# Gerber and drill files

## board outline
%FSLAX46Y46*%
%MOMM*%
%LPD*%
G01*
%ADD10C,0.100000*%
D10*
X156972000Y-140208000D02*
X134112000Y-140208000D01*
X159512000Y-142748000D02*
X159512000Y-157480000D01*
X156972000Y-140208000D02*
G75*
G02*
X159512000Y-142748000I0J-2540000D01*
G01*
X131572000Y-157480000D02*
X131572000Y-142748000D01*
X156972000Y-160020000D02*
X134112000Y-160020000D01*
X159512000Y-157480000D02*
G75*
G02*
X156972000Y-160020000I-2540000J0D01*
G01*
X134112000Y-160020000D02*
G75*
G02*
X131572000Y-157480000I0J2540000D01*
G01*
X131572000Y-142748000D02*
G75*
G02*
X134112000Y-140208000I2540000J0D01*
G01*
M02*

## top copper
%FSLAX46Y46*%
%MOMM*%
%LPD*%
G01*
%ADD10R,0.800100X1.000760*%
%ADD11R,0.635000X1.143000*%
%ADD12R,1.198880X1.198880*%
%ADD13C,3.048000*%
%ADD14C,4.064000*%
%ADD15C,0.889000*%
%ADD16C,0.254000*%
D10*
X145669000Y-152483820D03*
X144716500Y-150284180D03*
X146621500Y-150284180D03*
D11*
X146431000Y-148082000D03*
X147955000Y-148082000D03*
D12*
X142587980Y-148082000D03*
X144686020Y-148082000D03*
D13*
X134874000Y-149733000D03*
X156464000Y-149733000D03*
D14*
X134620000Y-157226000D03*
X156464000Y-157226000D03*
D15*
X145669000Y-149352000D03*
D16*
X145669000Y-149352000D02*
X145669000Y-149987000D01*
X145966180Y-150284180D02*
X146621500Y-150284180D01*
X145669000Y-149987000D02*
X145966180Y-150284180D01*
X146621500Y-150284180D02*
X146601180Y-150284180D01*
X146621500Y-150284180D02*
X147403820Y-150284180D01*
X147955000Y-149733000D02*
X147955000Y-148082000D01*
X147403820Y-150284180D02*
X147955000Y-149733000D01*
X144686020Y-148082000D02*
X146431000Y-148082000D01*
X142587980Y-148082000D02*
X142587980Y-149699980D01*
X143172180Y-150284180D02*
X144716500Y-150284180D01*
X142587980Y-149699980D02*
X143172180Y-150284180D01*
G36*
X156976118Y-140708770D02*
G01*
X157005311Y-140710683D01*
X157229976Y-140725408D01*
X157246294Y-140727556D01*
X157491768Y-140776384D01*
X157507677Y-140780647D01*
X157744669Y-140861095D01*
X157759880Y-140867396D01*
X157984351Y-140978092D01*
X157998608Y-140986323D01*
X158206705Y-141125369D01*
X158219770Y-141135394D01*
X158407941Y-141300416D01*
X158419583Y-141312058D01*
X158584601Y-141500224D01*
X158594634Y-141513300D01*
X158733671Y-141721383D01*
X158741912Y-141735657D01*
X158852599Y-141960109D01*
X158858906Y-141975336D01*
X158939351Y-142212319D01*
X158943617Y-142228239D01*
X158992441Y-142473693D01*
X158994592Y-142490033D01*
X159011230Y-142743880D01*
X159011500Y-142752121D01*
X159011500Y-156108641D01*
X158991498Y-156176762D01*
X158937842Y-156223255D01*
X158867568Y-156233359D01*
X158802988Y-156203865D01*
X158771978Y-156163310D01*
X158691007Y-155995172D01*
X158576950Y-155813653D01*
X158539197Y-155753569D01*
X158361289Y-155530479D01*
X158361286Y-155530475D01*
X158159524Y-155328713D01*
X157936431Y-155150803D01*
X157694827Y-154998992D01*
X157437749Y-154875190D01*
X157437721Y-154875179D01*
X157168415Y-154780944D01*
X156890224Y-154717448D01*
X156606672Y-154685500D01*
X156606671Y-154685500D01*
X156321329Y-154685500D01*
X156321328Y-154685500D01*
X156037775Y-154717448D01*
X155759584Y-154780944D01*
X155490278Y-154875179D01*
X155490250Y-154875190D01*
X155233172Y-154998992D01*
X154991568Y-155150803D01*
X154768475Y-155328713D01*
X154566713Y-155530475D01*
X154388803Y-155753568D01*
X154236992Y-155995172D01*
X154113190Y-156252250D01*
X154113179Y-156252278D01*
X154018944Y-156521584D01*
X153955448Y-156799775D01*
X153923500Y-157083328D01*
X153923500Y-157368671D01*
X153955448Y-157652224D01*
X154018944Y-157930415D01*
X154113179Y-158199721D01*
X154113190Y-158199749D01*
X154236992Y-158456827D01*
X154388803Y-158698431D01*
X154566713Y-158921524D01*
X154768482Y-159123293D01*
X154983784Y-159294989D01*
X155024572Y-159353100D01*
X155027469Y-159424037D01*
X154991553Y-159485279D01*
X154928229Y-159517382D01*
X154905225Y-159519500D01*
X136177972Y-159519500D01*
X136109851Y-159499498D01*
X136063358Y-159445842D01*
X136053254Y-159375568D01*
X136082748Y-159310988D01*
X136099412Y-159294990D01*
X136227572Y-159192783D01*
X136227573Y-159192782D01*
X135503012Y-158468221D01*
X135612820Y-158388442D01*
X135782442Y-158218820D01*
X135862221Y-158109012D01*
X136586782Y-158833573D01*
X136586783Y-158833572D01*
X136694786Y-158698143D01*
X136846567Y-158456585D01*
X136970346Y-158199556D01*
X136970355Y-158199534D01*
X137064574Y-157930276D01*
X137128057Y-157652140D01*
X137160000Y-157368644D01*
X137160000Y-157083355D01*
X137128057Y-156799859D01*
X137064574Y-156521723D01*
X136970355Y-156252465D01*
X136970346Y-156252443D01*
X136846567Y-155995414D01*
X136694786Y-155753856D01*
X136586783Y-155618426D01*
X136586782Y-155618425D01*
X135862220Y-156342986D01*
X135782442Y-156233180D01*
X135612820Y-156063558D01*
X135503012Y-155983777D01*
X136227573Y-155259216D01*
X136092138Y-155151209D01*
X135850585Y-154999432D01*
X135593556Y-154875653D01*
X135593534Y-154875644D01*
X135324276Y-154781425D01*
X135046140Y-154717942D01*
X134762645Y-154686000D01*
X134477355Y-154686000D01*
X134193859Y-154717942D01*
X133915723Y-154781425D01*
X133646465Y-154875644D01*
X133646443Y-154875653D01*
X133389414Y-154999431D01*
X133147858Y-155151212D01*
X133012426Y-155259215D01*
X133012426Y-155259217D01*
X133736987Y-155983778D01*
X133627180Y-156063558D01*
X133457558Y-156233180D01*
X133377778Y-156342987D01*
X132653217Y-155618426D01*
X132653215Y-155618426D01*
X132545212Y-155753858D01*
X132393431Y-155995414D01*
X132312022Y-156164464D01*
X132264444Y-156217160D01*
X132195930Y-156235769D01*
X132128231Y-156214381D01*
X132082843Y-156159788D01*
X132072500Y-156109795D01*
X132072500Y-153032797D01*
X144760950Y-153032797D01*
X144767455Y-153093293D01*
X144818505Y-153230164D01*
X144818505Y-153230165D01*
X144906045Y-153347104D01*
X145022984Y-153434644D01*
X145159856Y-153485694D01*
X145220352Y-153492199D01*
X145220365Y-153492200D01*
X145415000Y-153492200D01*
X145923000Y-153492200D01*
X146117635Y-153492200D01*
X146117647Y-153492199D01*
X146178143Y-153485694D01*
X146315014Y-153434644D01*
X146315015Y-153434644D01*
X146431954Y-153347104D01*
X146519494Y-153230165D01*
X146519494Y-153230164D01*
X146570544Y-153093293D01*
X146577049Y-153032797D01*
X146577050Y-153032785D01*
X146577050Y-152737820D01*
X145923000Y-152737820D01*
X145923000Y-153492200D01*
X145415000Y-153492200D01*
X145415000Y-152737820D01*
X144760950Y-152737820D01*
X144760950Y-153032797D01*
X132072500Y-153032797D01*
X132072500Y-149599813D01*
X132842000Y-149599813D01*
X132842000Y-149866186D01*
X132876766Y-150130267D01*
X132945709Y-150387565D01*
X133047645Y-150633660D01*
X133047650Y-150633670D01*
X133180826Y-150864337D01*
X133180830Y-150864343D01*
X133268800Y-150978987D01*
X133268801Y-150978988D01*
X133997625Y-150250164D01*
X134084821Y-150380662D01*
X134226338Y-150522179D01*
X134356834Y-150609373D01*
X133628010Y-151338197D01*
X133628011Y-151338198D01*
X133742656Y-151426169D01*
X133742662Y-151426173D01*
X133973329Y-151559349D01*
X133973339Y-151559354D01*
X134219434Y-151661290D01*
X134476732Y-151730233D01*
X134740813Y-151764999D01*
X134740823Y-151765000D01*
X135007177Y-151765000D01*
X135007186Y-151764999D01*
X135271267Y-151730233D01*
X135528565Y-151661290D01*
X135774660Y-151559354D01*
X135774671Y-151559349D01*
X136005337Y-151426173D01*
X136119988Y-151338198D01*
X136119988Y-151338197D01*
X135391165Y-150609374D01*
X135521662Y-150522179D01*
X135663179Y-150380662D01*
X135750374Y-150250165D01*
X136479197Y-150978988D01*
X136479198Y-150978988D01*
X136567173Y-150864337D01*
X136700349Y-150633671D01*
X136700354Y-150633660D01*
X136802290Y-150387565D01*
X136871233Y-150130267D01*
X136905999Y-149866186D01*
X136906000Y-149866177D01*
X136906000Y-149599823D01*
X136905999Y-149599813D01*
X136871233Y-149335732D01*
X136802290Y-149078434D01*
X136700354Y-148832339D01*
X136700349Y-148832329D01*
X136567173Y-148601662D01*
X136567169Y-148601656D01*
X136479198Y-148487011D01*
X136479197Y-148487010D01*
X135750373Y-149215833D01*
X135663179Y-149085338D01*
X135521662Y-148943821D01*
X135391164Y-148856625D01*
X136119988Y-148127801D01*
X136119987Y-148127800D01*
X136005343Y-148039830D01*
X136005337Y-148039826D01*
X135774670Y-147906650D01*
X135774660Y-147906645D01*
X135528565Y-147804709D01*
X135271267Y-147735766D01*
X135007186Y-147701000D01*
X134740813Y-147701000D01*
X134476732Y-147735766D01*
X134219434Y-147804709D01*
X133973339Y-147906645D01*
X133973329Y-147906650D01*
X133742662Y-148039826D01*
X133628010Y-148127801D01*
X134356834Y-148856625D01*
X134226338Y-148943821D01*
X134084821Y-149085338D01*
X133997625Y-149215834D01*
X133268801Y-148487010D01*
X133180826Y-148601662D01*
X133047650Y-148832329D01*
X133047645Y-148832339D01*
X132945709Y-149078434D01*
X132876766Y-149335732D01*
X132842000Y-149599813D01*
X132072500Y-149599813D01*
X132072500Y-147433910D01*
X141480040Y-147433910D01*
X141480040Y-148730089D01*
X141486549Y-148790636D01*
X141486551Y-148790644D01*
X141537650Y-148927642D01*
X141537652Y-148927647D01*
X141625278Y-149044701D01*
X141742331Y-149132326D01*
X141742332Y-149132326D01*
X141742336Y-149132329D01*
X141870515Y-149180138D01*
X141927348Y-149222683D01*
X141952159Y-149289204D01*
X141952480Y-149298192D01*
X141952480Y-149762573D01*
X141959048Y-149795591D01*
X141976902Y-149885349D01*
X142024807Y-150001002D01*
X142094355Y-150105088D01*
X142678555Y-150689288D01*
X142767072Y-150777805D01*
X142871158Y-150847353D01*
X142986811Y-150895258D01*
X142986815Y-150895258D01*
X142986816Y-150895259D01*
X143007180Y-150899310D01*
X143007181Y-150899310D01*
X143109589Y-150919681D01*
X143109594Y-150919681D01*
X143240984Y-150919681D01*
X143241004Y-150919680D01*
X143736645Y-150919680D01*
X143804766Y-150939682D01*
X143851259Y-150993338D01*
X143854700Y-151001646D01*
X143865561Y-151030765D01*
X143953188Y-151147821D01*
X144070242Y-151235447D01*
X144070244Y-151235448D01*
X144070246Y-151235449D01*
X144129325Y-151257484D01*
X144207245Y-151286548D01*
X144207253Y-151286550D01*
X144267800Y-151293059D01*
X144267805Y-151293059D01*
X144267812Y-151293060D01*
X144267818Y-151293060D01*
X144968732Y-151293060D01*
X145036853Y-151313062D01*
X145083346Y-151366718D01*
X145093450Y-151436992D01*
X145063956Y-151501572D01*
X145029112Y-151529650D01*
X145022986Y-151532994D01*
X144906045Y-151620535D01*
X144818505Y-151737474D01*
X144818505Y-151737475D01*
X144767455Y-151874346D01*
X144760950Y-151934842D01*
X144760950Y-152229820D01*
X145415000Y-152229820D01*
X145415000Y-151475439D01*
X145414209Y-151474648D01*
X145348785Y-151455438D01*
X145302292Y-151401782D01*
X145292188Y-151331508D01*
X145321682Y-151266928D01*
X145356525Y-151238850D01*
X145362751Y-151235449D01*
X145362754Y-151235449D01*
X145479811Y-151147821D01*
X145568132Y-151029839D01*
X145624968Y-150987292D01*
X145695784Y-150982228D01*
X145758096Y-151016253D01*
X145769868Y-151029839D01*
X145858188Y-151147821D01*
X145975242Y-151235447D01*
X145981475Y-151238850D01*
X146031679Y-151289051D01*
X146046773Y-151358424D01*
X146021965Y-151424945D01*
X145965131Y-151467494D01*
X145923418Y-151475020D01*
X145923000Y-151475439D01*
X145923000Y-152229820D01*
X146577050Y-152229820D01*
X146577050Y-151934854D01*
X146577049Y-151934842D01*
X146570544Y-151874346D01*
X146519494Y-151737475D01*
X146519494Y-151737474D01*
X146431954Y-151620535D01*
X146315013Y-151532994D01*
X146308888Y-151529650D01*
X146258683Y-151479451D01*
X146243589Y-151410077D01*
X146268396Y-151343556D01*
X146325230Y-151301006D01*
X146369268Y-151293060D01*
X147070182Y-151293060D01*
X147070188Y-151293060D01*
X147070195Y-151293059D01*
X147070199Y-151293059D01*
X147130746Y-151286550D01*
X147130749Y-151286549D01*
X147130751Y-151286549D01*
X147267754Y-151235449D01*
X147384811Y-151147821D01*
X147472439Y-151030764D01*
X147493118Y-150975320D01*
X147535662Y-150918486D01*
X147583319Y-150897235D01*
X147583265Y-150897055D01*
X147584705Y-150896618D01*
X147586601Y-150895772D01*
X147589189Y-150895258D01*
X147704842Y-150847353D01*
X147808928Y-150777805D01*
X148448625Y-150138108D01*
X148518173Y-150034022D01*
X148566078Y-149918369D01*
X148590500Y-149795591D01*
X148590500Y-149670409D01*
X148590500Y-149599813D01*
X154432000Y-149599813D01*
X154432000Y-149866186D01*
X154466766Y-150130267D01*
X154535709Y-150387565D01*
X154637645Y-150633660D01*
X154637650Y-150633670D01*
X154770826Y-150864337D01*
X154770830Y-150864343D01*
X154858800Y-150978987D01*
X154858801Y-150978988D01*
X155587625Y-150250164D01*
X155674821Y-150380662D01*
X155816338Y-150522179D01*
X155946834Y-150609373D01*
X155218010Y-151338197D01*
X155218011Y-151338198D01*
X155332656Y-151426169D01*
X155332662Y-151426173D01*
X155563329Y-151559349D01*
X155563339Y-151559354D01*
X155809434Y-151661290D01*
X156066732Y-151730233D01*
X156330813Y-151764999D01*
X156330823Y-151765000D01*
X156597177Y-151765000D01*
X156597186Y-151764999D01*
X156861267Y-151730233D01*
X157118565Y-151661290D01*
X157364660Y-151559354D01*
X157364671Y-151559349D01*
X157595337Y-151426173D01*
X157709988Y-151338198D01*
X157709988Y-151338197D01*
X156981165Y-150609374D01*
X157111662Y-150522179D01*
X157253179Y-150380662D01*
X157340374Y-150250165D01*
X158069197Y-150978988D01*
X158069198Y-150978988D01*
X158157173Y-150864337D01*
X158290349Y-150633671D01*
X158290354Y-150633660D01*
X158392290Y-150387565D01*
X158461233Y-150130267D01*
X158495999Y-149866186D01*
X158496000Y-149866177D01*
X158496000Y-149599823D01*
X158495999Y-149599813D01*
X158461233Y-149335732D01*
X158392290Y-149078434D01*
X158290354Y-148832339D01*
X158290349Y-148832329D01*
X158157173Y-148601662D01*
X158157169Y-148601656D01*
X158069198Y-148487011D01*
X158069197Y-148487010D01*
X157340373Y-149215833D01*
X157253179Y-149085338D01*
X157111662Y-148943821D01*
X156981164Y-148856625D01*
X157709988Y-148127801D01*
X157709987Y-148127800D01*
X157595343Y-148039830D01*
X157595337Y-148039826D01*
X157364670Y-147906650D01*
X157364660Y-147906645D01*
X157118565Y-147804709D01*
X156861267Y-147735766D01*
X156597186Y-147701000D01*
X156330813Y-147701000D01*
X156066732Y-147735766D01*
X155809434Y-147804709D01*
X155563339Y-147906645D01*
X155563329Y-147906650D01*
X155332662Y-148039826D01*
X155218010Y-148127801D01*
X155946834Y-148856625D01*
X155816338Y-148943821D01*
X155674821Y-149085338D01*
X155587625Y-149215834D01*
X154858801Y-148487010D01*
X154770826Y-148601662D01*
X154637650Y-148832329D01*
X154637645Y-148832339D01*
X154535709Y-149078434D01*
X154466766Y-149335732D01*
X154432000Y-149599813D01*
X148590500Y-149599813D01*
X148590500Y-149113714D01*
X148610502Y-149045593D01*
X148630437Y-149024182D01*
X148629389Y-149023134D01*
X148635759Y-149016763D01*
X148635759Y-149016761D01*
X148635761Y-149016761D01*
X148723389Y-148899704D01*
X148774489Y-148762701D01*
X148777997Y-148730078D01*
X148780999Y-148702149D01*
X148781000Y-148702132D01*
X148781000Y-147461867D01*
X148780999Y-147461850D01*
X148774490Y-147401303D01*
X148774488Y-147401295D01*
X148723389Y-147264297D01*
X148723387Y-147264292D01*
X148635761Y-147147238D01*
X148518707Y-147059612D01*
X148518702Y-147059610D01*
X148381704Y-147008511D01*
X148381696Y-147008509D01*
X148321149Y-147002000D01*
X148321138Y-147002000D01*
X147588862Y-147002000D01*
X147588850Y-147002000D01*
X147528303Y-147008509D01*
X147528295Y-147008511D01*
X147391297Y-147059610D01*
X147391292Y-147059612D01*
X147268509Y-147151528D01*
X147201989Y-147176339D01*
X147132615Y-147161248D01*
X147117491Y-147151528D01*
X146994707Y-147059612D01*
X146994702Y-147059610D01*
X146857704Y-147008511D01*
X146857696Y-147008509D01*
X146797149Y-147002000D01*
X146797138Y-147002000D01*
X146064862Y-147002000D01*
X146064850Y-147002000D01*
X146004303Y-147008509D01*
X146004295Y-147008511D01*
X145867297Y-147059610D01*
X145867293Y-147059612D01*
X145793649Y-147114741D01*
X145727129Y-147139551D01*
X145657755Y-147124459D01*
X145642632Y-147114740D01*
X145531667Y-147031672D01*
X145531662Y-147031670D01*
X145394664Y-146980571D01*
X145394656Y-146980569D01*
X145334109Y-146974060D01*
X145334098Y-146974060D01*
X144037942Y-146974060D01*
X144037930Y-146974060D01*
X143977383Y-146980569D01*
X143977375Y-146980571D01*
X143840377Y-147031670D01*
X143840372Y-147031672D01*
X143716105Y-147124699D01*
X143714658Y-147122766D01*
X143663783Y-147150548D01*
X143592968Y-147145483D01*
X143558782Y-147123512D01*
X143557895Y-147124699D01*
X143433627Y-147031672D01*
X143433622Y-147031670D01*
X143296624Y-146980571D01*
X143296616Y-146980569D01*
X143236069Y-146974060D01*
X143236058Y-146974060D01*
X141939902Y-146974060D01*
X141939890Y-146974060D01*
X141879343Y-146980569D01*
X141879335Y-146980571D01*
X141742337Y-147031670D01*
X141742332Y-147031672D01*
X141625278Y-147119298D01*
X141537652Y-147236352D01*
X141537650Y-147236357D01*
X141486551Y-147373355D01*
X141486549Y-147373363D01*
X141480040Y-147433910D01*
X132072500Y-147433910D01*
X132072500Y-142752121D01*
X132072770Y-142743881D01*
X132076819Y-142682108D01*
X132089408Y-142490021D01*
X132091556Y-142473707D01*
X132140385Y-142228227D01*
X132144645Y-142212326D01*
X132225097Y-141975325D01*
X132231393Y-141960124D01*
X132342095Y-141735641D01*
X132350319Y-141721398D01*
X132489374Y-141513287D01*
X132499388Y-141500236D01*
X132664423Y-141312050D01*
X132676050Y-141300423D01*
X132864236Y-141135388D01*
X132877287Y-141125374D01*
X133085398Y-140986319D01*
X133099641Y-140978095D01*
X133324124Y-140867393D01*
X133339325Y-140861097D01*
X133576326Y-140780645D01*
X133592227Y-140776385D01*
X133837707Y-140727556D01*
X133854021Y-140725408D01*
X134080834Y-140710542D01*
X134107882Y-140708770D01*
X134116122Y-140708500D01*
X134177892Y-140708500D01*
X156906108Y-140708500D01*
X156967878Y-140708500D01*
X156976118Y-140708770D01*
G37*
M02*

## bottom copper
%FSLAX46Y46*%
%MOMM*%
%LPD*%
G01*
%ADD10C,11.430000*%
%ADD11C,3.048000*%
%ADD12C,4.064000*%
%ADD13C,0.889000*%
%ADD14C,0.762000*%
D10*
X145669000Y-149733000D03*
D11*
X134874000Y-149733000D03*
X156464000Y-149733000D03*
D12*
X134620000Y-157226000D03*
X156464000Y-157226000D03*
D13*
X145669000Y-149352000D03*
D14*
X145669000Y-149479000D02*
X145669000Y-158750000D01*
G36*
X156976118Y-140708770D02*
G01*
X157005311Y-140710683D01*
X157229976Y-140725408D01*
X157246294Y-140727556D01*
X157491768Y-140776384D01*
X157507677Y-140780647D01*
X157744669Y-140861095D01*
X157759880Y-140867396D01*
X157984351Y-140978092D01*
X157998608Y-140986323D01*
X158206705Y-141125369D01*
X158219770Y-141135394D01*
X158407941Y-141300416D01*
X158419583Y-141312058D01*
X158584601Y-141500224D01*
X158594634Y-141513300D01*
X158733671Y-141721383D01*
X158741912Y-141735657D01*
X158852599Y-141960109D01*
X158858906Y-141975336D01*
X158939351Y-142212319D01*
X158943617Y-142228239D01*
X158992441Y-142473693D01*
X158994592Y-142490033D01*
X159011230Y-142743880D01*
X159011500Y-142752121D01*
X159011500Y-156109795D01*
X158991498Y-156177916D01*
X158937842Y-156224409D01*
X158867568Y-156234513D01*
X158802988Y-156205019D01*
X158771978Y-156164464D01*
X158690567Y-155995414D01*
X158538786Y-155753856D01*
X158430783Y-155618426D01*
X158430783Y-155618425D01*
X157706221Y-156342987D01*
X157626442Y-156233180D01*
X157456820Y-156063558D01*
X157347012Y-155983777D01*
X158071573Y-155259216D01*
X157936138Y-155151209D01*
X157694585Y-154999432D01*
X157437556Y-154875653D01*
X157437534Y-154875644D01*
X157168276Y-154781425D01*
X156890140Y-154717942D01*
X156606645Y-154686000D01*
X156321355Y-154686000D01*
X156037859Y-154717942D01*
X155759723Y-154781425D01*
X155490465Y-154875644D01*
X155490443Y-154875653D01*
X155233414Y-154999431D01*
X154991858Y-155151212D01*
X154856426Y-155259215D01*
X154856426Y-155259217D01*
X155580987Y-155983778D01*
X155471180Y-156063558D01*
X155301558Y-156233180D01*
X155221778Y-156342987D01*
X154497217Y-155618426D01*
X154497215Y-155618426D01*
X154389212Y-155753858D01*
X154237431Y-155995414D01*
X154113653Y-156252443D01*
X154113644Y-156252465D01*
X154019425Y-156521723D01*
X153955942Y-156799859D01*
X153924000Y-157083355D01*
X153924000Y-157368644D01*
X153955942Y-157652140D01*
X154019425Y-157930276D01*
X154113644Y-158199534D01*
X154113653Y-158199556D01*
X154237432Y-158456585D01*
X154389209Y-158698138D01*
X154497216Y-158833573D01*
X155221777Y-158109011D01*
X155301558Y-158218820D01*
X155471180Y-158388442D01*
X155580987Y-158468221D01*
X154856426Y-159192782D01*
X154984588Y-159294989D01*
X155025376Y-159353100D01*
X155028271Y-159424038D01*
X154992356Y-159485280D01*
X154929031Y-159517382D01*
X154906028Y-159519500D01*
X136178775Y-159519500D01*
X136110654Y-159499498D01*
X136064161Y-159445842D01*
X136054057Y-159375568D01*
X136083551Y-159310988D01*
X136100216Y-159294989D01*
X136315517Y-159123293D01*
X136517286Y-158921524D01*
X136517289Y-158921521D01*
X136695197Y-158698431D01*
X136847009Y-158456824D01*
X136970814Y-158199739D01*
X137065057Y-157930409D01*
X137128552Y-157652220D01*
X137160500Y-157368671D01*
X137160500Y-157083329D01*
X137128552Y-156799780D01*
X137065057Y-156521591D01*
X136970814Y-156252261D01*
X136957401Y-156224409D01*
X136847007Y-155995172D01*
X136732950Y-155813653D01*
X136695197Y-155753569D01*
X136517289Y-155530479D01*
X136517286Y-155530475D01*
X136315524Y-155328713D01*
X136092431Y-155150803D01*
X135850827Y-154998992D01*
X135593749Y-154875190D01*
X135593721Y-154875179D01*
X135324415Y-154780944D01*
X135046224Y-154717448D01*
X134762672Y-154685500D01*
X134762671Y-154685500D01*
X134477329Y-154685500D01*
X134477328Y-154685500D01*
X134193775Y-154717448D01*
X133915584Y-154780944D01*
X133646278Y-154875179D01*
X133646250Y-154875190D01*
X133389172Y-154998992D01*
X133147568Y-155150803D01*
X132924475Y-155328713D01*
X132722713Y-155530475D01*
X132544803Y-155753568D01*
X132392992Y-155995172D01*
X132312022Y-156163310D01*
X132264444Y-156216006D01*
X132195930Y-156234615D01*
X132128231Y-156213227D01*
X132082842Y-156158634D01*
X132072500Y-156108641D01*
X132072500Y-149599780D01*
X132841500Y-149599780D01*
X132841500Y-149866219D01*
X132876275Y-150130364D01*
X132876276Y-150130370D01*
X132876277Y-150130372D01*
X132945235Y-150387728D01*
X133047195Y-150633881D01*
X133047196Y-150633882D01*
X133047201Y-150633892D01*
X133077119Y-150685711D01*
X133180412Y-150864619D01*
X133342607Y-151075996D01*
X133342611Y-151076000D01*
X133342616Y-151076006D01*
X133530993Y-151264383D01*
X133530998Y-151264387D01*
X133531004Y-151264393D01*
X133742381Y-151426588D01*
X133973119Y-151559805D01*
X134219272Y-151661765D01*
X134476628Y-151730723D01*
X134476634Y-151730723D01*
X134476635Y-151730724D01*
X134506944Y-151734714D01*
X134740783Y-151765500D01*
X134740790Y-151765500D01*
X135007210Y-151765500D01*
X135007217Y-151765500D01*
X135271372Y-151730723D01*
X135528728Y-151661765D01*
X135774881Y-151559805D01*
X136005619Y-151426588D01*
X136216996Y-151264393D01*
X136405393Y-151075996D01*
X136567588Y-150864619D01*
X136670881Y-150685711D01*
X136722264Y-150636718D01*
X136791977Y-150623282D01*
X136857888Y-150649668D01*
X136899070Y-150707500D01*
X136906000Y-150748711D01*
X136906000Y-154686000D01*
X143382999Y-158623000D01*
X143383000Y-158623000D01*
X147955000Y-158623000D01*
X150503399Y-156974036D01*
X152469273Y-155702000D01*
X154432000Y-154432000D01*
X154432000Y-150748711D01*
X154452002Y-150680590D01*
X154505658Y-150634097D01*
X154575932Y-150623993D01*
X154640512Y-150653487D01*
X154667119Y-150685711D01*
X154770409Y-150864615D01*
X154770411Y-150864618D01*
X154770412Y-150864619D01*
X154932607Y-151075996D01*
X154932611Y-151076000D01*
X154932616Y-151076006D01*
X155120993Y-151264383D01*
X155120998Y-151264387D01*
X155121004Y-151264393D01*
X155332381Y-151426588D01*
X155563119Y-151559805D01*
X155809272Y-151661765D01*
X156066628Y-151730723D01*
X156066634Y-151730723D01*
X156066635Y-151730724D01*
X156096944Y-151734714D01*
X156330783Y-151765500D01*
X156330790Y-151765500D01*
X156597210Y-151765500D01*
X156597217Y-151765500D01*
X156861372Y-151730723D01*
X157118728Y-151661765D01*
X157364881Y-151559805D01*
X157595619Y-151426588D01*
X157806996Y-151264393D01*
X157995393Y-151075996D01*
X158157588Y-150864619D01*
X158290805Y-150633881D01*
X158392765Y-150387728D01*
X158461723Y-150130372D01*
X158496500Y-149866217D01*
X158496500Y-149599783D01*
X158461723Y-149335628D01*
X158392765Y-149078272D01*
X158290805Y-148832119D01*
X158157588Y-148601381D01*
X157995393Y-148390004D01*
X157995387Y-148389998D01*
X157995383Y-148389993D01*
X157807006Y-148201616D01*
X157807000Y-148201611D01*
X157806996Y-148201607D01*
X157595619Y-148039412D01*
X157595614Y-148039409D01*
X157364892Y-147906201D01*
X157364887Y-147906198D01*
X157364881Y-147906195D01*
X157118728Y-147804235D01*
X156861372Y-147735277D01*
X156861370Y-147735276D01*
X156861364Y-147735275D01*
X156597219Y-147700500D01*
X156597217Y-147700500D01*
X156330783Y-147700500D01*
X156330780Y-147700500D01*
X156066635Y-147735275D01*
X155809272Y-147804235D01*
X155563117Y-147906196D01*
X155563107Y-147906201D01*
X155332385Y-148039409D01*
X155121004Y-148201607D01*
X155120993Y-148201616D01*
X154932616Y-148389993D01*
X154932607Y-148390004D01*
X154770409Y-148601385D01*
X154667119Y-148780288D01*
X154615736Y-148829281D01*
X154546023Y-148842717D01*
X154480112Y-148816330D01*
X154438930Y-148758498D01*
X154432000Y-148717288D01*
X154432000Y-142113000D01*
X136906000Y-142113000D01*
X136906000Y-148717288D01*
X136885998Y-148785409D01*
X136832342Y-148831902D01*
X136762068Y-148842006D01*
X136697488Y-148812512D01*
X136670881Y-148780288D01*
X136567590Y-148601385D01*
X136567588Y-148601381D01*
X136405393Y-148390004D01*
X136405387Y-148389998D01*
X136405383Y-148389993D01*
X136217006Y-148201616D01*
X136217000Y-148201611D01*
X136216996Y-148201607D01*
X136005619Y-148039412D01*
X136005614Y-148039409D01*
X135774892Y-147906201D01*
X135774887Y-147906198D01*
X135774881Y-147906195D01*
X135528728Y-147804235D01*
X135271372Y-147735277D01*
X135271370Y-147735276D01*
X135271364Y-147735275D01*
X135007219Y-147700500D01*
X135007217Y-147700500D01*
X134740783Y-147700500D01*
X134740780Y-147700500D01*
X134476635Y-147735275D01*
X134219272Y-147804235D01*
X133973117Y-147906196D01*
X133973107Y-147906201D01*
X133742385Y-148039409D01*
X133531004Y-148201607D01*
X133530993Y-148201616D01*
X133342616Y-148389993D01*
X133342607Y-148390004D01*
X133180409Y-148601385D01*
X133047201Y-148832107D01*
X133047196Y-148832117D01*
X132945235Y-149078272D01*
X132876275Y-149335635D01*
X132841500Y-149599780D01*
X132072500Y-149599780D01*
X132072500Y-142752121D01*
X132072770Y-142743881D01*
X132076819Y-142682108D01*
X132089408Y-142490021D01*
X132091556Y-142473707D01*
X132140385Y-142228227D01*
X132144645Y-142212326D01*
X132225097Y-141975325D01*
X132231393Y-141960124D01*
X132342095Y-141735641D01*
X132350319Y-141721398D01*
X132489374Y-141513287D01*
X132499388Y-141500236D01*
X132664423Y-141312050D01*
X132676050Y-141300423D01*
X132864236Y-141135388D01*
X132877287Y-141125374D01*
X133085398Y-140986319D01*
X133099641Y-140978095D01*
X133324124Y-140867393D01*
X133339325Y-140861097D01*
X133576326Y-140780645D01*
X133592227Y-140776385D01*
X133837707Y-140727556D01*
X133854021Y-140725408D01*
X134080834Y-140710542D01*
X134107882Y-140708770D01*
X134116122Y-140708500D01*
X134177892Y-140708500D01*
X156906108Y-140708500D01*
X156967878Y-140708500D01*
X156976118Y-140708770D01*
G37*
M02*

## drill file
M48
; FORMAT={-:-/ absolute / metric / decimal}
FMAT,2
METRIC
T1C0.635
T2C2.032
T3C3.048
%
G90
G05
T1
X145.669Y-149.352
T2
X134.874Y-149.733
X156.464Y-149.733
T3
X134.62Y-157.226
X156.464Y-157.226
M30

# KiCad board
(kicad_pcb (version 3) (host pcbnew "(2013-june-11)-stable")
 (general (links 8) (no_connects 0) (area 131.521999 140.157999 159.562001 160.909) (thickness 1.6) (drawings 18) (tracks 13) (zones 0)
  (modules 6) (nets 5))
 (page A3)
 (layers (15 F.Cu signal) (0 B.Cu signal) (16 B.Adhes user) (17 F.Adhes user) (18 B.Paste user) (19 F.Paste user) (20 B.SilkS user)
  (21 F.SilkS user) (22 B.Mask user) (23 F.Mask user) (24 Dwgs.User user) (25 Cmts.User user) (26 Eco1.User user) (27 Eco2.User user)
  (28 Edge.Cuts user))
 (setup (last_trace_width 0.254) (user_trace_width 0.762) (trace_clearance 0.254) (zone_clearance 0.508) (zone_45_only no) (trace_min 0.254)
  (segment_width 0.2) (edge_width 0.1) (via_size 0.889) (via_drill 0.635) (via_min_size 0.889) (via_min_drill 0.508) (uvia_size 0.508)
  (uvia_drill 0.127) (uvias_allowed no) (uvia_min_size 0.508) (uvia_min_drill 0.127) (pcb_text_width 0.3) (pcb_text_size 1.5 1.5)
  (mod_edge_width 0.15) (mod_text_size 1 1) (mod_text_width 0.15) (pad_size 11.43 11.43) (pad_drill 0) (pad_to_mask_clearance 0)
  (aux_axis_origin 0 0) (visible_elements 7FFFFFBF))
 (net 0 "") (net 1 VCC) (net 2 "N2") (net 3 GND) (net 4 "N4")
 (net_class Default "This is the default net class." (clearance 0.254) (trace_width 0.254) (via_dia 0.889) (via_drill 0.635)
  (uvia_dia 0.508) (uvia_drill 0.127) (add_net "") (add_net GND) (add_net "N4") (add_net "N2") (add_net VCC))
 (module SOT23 (layer F.Cu) (at 145.669 151.384 180)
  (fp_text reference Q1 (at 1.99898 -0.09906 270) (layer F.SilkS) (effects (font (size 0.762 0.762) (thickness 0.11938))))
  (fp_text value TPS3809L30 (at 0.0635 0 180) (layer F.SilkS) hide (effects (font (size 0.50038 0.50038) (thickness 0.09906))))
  (pad 3 smd rect (at 0 -1.09982 180) (size 0.8001 1.00076) (layers F.Cu F.Paste F.Mask) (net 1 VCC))
  (pad 2 smd rect (at 0.9525 1.09982 180) (size 0.8001 1.00076) (layers F.Cu F.Paste F.Mask) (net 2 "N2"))
  (pad 1 smd rect (at -0.9525 1.09982 180) (size 0.8001 1.00076) (layers F.Cu F.Paste F.Mask) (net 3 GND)))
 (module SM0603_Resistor (layer F.Cu) (at 147.193 148.082)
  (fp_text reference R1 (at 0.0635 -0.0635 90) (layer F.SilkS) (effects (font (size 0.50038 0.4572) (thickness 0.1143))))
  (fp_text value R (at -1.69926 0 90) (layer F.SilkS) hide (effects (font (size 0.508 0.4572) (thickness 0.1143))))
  (pad 1 smd rect (at -0.762 0) (size 0.635 1.143) (layers F.Cu F.Paste F.Mask) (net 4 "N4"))
  (pad 2 smd rect (at 0.762 0) (size 0.635 1.143) (layers F.Cu F.Paste F.Mask) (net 3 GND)))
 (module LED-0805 (layer F.Cu) (at 143.637 148.082)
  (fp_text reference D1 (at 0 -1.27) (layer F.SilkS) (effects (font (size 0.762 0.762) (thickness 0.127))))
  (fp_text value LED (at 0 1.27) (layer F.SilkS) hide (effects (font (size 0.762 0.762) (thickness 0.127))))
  (pad 1 smd rect (at -1.04902 0) (size 1.19888 1.19888) (layers F.Cu F.Paste F.Mask) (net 2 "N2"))
  (pad 2 smd rect (at 1.04902 0) (size 1.19888 1.19888) (layers F.Cu F.Paste F.Mask) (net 4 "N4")))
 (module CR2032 (layer B.Cu) (at 145.669 149.733 180)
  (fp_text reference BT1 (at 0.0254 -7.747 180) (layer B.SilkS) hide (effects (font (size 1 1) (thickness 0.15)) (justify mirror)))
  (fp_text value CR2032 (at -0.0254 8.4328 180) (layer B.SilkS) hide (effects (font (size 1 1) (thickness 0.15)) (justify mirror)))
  (pad 2 smd circle (at 0 0 180) (size 11.43 11.43) (layers B.Cu B.Paste B.Mask) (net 3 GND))
  (pad 1 thru_hole circle (at 10.795 0 180) (size 3.048 3.048) (drill 2.032) (layers *.Cu *.Mask B.SilkS) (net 1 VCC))
  (pad 1 thru_hole circle (at -10.795 0 180) (size 3.048 3.048) (drill 2.032) (layers *.Cu *.Mask B.SilkS) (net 1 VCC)))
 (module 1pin (layer F.Cu) (at 134.62 157.226)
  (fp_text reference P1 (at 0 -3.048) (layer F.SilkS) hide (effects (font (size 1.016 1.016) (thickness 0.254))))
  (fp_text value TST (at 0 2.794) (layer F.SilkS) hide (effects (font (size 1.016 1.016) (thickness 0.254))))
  (pad 1 thru_hole circle (at 0 0) (size 4.064 4.064) (drill 3.048) (layers *.Cu *.Mask F.SilkS) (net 1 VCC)))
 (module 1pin (layer F.Cu) (at 156.464 157.226)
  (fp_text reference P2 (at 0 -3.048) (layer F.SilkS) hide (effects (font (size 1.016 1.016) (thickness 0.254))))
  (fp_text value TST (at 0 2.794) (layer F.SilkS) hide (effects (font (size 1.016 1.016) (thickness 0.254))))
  (pad 1 thru_hole circle (at 0 0) (size 4.064 4.064) (drill 3.048) (layers *.Cu *.Mask F.SilkS) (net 3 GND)))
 (gr_line (start 156.972 140.208) (end 134.112 140.208) (angle 90) (layer Edge.Cuts) (width 0.1))
 (gr_line (start 159.512 142.748) (end 159.512 157.48) (angle 90) (layer Edge.Cuts) (width 0.1))
 (gr_arc (start 156.972 142.748) (end 156.972 140.208) (angle 90) (layer Edge.Cuts) (width 0.1))
 (gr_line (start 131.572 157.48) (end 131.572 142.748) (angle 90) (layer Edge.Cuts) (width 0.1))
 (gr_line (start 156.972 160.02) (end 134.112 160.02) (angle 90) (layer Edge.Cuts) (width 0.1))
 (gr_arc (start 156.972 157.48) (end 159.512 157.48) (angle 90) (layer Edge.Cuts) (width 0.1))
 (gr_arc (start 134.112 157.48) (end 134.112 160.02) (angle 90) (layer Edge.Cuts) (width 0.1))
 (gr_arc (start 134.112 142.748) (end 131.572 142.748) (angle 90) (layer Edge.Cuts) (width 0.1))
 (segment (start 145.669 149.479) (end 145.669 158.75) (width 0.762) (layer B.Cu) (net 3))
 (segment (start 145.669 149.352) (end 145.669 149.987) (width 0.254) (layer F.Cu) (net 3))
 (via (at 145.669 149.352) (size 0.889) (layers F.Cu B.Cu) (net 3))
 (segment (start 145.96618 150.28418) (end 146.6215 150.28418) (width 0.254) (layer F.Cu) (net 3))
 (segment (start 145.669 149.987) (end 145.96618 150.28418) (width 0.254) (layer F.Cu) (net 3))
 (segment (start 146.6215 150.28418) (end 146.60118 150.28418) (width 0.254) (layer F.Cu) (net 3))
 (segment (start 146.6215 150.28418) (end 147.40382 150.28418) (width 0.254) (layer F.Cu) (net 3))
 (segment (start 147.955 149.733) (end 147.955 148.082) (width 0.254) (layer F.Cu) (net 3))
 (segment (start 147.40382 150.28418) (end 147.955 149.733) (width 0.254) (layer F.Cu) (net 3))
 (segment (start 144.68602 148.082) (end 146.431 148.082) (width 0.254) (layer F.Cu) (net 4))
 (segment (start 142.58798 148.082) (end 142.58798 149.69998) (width 0.254) (layer F.Cu) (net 2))
 (segment (start 143.17218 150.28418) (end 144.7165 150.28418) (width 0.254) (layer F.Cu) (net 2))
 (segment (start 142.58798 149.69998) (end 143.17218 150.28418) (width 0.254) (layer F.Cu) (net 2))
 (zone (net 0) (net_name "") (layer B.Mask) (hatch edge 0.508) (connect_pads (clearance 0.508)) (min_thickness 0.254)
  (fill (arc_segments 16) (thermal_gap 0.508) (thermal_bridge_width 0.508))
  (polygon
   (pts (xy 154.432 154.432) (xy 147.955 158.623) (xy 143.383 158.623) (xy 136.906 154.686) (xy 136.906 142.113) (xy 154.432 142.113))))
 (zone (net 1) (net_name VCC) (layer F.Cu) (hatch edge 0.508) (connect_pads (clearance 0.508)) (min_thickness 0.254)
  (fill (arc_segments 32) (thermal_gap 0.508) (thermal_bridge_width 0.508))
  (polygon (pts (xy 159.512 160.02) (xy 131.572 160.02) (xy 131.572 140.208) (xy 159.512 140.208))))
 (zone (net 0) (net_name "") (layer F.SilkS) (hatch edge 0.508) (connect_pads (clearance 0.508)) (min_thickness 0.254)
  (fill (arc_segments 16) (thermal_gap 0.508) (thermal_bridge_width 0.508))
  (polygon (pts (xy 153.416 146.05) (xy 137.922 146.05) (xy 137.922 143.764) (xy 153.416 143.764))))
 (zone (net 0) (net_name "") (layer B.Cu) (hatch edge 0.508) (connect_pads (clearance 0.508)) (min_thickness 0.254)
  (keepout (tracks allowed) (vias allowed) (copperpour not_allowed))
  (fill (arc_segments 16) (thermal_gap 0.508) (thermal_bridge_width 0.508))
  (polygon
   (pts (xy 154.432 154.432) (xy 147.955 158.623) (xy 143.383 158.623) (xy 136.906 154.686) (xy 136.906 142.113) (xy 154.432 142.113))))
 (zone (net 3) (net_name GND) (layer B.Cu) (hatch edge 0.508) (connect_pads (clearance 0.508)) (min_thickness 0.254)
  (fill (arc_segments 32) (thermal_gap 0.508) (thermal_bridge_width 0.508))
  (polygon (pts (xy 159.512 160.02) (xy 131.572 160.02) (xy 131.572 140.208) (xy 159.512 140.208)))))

